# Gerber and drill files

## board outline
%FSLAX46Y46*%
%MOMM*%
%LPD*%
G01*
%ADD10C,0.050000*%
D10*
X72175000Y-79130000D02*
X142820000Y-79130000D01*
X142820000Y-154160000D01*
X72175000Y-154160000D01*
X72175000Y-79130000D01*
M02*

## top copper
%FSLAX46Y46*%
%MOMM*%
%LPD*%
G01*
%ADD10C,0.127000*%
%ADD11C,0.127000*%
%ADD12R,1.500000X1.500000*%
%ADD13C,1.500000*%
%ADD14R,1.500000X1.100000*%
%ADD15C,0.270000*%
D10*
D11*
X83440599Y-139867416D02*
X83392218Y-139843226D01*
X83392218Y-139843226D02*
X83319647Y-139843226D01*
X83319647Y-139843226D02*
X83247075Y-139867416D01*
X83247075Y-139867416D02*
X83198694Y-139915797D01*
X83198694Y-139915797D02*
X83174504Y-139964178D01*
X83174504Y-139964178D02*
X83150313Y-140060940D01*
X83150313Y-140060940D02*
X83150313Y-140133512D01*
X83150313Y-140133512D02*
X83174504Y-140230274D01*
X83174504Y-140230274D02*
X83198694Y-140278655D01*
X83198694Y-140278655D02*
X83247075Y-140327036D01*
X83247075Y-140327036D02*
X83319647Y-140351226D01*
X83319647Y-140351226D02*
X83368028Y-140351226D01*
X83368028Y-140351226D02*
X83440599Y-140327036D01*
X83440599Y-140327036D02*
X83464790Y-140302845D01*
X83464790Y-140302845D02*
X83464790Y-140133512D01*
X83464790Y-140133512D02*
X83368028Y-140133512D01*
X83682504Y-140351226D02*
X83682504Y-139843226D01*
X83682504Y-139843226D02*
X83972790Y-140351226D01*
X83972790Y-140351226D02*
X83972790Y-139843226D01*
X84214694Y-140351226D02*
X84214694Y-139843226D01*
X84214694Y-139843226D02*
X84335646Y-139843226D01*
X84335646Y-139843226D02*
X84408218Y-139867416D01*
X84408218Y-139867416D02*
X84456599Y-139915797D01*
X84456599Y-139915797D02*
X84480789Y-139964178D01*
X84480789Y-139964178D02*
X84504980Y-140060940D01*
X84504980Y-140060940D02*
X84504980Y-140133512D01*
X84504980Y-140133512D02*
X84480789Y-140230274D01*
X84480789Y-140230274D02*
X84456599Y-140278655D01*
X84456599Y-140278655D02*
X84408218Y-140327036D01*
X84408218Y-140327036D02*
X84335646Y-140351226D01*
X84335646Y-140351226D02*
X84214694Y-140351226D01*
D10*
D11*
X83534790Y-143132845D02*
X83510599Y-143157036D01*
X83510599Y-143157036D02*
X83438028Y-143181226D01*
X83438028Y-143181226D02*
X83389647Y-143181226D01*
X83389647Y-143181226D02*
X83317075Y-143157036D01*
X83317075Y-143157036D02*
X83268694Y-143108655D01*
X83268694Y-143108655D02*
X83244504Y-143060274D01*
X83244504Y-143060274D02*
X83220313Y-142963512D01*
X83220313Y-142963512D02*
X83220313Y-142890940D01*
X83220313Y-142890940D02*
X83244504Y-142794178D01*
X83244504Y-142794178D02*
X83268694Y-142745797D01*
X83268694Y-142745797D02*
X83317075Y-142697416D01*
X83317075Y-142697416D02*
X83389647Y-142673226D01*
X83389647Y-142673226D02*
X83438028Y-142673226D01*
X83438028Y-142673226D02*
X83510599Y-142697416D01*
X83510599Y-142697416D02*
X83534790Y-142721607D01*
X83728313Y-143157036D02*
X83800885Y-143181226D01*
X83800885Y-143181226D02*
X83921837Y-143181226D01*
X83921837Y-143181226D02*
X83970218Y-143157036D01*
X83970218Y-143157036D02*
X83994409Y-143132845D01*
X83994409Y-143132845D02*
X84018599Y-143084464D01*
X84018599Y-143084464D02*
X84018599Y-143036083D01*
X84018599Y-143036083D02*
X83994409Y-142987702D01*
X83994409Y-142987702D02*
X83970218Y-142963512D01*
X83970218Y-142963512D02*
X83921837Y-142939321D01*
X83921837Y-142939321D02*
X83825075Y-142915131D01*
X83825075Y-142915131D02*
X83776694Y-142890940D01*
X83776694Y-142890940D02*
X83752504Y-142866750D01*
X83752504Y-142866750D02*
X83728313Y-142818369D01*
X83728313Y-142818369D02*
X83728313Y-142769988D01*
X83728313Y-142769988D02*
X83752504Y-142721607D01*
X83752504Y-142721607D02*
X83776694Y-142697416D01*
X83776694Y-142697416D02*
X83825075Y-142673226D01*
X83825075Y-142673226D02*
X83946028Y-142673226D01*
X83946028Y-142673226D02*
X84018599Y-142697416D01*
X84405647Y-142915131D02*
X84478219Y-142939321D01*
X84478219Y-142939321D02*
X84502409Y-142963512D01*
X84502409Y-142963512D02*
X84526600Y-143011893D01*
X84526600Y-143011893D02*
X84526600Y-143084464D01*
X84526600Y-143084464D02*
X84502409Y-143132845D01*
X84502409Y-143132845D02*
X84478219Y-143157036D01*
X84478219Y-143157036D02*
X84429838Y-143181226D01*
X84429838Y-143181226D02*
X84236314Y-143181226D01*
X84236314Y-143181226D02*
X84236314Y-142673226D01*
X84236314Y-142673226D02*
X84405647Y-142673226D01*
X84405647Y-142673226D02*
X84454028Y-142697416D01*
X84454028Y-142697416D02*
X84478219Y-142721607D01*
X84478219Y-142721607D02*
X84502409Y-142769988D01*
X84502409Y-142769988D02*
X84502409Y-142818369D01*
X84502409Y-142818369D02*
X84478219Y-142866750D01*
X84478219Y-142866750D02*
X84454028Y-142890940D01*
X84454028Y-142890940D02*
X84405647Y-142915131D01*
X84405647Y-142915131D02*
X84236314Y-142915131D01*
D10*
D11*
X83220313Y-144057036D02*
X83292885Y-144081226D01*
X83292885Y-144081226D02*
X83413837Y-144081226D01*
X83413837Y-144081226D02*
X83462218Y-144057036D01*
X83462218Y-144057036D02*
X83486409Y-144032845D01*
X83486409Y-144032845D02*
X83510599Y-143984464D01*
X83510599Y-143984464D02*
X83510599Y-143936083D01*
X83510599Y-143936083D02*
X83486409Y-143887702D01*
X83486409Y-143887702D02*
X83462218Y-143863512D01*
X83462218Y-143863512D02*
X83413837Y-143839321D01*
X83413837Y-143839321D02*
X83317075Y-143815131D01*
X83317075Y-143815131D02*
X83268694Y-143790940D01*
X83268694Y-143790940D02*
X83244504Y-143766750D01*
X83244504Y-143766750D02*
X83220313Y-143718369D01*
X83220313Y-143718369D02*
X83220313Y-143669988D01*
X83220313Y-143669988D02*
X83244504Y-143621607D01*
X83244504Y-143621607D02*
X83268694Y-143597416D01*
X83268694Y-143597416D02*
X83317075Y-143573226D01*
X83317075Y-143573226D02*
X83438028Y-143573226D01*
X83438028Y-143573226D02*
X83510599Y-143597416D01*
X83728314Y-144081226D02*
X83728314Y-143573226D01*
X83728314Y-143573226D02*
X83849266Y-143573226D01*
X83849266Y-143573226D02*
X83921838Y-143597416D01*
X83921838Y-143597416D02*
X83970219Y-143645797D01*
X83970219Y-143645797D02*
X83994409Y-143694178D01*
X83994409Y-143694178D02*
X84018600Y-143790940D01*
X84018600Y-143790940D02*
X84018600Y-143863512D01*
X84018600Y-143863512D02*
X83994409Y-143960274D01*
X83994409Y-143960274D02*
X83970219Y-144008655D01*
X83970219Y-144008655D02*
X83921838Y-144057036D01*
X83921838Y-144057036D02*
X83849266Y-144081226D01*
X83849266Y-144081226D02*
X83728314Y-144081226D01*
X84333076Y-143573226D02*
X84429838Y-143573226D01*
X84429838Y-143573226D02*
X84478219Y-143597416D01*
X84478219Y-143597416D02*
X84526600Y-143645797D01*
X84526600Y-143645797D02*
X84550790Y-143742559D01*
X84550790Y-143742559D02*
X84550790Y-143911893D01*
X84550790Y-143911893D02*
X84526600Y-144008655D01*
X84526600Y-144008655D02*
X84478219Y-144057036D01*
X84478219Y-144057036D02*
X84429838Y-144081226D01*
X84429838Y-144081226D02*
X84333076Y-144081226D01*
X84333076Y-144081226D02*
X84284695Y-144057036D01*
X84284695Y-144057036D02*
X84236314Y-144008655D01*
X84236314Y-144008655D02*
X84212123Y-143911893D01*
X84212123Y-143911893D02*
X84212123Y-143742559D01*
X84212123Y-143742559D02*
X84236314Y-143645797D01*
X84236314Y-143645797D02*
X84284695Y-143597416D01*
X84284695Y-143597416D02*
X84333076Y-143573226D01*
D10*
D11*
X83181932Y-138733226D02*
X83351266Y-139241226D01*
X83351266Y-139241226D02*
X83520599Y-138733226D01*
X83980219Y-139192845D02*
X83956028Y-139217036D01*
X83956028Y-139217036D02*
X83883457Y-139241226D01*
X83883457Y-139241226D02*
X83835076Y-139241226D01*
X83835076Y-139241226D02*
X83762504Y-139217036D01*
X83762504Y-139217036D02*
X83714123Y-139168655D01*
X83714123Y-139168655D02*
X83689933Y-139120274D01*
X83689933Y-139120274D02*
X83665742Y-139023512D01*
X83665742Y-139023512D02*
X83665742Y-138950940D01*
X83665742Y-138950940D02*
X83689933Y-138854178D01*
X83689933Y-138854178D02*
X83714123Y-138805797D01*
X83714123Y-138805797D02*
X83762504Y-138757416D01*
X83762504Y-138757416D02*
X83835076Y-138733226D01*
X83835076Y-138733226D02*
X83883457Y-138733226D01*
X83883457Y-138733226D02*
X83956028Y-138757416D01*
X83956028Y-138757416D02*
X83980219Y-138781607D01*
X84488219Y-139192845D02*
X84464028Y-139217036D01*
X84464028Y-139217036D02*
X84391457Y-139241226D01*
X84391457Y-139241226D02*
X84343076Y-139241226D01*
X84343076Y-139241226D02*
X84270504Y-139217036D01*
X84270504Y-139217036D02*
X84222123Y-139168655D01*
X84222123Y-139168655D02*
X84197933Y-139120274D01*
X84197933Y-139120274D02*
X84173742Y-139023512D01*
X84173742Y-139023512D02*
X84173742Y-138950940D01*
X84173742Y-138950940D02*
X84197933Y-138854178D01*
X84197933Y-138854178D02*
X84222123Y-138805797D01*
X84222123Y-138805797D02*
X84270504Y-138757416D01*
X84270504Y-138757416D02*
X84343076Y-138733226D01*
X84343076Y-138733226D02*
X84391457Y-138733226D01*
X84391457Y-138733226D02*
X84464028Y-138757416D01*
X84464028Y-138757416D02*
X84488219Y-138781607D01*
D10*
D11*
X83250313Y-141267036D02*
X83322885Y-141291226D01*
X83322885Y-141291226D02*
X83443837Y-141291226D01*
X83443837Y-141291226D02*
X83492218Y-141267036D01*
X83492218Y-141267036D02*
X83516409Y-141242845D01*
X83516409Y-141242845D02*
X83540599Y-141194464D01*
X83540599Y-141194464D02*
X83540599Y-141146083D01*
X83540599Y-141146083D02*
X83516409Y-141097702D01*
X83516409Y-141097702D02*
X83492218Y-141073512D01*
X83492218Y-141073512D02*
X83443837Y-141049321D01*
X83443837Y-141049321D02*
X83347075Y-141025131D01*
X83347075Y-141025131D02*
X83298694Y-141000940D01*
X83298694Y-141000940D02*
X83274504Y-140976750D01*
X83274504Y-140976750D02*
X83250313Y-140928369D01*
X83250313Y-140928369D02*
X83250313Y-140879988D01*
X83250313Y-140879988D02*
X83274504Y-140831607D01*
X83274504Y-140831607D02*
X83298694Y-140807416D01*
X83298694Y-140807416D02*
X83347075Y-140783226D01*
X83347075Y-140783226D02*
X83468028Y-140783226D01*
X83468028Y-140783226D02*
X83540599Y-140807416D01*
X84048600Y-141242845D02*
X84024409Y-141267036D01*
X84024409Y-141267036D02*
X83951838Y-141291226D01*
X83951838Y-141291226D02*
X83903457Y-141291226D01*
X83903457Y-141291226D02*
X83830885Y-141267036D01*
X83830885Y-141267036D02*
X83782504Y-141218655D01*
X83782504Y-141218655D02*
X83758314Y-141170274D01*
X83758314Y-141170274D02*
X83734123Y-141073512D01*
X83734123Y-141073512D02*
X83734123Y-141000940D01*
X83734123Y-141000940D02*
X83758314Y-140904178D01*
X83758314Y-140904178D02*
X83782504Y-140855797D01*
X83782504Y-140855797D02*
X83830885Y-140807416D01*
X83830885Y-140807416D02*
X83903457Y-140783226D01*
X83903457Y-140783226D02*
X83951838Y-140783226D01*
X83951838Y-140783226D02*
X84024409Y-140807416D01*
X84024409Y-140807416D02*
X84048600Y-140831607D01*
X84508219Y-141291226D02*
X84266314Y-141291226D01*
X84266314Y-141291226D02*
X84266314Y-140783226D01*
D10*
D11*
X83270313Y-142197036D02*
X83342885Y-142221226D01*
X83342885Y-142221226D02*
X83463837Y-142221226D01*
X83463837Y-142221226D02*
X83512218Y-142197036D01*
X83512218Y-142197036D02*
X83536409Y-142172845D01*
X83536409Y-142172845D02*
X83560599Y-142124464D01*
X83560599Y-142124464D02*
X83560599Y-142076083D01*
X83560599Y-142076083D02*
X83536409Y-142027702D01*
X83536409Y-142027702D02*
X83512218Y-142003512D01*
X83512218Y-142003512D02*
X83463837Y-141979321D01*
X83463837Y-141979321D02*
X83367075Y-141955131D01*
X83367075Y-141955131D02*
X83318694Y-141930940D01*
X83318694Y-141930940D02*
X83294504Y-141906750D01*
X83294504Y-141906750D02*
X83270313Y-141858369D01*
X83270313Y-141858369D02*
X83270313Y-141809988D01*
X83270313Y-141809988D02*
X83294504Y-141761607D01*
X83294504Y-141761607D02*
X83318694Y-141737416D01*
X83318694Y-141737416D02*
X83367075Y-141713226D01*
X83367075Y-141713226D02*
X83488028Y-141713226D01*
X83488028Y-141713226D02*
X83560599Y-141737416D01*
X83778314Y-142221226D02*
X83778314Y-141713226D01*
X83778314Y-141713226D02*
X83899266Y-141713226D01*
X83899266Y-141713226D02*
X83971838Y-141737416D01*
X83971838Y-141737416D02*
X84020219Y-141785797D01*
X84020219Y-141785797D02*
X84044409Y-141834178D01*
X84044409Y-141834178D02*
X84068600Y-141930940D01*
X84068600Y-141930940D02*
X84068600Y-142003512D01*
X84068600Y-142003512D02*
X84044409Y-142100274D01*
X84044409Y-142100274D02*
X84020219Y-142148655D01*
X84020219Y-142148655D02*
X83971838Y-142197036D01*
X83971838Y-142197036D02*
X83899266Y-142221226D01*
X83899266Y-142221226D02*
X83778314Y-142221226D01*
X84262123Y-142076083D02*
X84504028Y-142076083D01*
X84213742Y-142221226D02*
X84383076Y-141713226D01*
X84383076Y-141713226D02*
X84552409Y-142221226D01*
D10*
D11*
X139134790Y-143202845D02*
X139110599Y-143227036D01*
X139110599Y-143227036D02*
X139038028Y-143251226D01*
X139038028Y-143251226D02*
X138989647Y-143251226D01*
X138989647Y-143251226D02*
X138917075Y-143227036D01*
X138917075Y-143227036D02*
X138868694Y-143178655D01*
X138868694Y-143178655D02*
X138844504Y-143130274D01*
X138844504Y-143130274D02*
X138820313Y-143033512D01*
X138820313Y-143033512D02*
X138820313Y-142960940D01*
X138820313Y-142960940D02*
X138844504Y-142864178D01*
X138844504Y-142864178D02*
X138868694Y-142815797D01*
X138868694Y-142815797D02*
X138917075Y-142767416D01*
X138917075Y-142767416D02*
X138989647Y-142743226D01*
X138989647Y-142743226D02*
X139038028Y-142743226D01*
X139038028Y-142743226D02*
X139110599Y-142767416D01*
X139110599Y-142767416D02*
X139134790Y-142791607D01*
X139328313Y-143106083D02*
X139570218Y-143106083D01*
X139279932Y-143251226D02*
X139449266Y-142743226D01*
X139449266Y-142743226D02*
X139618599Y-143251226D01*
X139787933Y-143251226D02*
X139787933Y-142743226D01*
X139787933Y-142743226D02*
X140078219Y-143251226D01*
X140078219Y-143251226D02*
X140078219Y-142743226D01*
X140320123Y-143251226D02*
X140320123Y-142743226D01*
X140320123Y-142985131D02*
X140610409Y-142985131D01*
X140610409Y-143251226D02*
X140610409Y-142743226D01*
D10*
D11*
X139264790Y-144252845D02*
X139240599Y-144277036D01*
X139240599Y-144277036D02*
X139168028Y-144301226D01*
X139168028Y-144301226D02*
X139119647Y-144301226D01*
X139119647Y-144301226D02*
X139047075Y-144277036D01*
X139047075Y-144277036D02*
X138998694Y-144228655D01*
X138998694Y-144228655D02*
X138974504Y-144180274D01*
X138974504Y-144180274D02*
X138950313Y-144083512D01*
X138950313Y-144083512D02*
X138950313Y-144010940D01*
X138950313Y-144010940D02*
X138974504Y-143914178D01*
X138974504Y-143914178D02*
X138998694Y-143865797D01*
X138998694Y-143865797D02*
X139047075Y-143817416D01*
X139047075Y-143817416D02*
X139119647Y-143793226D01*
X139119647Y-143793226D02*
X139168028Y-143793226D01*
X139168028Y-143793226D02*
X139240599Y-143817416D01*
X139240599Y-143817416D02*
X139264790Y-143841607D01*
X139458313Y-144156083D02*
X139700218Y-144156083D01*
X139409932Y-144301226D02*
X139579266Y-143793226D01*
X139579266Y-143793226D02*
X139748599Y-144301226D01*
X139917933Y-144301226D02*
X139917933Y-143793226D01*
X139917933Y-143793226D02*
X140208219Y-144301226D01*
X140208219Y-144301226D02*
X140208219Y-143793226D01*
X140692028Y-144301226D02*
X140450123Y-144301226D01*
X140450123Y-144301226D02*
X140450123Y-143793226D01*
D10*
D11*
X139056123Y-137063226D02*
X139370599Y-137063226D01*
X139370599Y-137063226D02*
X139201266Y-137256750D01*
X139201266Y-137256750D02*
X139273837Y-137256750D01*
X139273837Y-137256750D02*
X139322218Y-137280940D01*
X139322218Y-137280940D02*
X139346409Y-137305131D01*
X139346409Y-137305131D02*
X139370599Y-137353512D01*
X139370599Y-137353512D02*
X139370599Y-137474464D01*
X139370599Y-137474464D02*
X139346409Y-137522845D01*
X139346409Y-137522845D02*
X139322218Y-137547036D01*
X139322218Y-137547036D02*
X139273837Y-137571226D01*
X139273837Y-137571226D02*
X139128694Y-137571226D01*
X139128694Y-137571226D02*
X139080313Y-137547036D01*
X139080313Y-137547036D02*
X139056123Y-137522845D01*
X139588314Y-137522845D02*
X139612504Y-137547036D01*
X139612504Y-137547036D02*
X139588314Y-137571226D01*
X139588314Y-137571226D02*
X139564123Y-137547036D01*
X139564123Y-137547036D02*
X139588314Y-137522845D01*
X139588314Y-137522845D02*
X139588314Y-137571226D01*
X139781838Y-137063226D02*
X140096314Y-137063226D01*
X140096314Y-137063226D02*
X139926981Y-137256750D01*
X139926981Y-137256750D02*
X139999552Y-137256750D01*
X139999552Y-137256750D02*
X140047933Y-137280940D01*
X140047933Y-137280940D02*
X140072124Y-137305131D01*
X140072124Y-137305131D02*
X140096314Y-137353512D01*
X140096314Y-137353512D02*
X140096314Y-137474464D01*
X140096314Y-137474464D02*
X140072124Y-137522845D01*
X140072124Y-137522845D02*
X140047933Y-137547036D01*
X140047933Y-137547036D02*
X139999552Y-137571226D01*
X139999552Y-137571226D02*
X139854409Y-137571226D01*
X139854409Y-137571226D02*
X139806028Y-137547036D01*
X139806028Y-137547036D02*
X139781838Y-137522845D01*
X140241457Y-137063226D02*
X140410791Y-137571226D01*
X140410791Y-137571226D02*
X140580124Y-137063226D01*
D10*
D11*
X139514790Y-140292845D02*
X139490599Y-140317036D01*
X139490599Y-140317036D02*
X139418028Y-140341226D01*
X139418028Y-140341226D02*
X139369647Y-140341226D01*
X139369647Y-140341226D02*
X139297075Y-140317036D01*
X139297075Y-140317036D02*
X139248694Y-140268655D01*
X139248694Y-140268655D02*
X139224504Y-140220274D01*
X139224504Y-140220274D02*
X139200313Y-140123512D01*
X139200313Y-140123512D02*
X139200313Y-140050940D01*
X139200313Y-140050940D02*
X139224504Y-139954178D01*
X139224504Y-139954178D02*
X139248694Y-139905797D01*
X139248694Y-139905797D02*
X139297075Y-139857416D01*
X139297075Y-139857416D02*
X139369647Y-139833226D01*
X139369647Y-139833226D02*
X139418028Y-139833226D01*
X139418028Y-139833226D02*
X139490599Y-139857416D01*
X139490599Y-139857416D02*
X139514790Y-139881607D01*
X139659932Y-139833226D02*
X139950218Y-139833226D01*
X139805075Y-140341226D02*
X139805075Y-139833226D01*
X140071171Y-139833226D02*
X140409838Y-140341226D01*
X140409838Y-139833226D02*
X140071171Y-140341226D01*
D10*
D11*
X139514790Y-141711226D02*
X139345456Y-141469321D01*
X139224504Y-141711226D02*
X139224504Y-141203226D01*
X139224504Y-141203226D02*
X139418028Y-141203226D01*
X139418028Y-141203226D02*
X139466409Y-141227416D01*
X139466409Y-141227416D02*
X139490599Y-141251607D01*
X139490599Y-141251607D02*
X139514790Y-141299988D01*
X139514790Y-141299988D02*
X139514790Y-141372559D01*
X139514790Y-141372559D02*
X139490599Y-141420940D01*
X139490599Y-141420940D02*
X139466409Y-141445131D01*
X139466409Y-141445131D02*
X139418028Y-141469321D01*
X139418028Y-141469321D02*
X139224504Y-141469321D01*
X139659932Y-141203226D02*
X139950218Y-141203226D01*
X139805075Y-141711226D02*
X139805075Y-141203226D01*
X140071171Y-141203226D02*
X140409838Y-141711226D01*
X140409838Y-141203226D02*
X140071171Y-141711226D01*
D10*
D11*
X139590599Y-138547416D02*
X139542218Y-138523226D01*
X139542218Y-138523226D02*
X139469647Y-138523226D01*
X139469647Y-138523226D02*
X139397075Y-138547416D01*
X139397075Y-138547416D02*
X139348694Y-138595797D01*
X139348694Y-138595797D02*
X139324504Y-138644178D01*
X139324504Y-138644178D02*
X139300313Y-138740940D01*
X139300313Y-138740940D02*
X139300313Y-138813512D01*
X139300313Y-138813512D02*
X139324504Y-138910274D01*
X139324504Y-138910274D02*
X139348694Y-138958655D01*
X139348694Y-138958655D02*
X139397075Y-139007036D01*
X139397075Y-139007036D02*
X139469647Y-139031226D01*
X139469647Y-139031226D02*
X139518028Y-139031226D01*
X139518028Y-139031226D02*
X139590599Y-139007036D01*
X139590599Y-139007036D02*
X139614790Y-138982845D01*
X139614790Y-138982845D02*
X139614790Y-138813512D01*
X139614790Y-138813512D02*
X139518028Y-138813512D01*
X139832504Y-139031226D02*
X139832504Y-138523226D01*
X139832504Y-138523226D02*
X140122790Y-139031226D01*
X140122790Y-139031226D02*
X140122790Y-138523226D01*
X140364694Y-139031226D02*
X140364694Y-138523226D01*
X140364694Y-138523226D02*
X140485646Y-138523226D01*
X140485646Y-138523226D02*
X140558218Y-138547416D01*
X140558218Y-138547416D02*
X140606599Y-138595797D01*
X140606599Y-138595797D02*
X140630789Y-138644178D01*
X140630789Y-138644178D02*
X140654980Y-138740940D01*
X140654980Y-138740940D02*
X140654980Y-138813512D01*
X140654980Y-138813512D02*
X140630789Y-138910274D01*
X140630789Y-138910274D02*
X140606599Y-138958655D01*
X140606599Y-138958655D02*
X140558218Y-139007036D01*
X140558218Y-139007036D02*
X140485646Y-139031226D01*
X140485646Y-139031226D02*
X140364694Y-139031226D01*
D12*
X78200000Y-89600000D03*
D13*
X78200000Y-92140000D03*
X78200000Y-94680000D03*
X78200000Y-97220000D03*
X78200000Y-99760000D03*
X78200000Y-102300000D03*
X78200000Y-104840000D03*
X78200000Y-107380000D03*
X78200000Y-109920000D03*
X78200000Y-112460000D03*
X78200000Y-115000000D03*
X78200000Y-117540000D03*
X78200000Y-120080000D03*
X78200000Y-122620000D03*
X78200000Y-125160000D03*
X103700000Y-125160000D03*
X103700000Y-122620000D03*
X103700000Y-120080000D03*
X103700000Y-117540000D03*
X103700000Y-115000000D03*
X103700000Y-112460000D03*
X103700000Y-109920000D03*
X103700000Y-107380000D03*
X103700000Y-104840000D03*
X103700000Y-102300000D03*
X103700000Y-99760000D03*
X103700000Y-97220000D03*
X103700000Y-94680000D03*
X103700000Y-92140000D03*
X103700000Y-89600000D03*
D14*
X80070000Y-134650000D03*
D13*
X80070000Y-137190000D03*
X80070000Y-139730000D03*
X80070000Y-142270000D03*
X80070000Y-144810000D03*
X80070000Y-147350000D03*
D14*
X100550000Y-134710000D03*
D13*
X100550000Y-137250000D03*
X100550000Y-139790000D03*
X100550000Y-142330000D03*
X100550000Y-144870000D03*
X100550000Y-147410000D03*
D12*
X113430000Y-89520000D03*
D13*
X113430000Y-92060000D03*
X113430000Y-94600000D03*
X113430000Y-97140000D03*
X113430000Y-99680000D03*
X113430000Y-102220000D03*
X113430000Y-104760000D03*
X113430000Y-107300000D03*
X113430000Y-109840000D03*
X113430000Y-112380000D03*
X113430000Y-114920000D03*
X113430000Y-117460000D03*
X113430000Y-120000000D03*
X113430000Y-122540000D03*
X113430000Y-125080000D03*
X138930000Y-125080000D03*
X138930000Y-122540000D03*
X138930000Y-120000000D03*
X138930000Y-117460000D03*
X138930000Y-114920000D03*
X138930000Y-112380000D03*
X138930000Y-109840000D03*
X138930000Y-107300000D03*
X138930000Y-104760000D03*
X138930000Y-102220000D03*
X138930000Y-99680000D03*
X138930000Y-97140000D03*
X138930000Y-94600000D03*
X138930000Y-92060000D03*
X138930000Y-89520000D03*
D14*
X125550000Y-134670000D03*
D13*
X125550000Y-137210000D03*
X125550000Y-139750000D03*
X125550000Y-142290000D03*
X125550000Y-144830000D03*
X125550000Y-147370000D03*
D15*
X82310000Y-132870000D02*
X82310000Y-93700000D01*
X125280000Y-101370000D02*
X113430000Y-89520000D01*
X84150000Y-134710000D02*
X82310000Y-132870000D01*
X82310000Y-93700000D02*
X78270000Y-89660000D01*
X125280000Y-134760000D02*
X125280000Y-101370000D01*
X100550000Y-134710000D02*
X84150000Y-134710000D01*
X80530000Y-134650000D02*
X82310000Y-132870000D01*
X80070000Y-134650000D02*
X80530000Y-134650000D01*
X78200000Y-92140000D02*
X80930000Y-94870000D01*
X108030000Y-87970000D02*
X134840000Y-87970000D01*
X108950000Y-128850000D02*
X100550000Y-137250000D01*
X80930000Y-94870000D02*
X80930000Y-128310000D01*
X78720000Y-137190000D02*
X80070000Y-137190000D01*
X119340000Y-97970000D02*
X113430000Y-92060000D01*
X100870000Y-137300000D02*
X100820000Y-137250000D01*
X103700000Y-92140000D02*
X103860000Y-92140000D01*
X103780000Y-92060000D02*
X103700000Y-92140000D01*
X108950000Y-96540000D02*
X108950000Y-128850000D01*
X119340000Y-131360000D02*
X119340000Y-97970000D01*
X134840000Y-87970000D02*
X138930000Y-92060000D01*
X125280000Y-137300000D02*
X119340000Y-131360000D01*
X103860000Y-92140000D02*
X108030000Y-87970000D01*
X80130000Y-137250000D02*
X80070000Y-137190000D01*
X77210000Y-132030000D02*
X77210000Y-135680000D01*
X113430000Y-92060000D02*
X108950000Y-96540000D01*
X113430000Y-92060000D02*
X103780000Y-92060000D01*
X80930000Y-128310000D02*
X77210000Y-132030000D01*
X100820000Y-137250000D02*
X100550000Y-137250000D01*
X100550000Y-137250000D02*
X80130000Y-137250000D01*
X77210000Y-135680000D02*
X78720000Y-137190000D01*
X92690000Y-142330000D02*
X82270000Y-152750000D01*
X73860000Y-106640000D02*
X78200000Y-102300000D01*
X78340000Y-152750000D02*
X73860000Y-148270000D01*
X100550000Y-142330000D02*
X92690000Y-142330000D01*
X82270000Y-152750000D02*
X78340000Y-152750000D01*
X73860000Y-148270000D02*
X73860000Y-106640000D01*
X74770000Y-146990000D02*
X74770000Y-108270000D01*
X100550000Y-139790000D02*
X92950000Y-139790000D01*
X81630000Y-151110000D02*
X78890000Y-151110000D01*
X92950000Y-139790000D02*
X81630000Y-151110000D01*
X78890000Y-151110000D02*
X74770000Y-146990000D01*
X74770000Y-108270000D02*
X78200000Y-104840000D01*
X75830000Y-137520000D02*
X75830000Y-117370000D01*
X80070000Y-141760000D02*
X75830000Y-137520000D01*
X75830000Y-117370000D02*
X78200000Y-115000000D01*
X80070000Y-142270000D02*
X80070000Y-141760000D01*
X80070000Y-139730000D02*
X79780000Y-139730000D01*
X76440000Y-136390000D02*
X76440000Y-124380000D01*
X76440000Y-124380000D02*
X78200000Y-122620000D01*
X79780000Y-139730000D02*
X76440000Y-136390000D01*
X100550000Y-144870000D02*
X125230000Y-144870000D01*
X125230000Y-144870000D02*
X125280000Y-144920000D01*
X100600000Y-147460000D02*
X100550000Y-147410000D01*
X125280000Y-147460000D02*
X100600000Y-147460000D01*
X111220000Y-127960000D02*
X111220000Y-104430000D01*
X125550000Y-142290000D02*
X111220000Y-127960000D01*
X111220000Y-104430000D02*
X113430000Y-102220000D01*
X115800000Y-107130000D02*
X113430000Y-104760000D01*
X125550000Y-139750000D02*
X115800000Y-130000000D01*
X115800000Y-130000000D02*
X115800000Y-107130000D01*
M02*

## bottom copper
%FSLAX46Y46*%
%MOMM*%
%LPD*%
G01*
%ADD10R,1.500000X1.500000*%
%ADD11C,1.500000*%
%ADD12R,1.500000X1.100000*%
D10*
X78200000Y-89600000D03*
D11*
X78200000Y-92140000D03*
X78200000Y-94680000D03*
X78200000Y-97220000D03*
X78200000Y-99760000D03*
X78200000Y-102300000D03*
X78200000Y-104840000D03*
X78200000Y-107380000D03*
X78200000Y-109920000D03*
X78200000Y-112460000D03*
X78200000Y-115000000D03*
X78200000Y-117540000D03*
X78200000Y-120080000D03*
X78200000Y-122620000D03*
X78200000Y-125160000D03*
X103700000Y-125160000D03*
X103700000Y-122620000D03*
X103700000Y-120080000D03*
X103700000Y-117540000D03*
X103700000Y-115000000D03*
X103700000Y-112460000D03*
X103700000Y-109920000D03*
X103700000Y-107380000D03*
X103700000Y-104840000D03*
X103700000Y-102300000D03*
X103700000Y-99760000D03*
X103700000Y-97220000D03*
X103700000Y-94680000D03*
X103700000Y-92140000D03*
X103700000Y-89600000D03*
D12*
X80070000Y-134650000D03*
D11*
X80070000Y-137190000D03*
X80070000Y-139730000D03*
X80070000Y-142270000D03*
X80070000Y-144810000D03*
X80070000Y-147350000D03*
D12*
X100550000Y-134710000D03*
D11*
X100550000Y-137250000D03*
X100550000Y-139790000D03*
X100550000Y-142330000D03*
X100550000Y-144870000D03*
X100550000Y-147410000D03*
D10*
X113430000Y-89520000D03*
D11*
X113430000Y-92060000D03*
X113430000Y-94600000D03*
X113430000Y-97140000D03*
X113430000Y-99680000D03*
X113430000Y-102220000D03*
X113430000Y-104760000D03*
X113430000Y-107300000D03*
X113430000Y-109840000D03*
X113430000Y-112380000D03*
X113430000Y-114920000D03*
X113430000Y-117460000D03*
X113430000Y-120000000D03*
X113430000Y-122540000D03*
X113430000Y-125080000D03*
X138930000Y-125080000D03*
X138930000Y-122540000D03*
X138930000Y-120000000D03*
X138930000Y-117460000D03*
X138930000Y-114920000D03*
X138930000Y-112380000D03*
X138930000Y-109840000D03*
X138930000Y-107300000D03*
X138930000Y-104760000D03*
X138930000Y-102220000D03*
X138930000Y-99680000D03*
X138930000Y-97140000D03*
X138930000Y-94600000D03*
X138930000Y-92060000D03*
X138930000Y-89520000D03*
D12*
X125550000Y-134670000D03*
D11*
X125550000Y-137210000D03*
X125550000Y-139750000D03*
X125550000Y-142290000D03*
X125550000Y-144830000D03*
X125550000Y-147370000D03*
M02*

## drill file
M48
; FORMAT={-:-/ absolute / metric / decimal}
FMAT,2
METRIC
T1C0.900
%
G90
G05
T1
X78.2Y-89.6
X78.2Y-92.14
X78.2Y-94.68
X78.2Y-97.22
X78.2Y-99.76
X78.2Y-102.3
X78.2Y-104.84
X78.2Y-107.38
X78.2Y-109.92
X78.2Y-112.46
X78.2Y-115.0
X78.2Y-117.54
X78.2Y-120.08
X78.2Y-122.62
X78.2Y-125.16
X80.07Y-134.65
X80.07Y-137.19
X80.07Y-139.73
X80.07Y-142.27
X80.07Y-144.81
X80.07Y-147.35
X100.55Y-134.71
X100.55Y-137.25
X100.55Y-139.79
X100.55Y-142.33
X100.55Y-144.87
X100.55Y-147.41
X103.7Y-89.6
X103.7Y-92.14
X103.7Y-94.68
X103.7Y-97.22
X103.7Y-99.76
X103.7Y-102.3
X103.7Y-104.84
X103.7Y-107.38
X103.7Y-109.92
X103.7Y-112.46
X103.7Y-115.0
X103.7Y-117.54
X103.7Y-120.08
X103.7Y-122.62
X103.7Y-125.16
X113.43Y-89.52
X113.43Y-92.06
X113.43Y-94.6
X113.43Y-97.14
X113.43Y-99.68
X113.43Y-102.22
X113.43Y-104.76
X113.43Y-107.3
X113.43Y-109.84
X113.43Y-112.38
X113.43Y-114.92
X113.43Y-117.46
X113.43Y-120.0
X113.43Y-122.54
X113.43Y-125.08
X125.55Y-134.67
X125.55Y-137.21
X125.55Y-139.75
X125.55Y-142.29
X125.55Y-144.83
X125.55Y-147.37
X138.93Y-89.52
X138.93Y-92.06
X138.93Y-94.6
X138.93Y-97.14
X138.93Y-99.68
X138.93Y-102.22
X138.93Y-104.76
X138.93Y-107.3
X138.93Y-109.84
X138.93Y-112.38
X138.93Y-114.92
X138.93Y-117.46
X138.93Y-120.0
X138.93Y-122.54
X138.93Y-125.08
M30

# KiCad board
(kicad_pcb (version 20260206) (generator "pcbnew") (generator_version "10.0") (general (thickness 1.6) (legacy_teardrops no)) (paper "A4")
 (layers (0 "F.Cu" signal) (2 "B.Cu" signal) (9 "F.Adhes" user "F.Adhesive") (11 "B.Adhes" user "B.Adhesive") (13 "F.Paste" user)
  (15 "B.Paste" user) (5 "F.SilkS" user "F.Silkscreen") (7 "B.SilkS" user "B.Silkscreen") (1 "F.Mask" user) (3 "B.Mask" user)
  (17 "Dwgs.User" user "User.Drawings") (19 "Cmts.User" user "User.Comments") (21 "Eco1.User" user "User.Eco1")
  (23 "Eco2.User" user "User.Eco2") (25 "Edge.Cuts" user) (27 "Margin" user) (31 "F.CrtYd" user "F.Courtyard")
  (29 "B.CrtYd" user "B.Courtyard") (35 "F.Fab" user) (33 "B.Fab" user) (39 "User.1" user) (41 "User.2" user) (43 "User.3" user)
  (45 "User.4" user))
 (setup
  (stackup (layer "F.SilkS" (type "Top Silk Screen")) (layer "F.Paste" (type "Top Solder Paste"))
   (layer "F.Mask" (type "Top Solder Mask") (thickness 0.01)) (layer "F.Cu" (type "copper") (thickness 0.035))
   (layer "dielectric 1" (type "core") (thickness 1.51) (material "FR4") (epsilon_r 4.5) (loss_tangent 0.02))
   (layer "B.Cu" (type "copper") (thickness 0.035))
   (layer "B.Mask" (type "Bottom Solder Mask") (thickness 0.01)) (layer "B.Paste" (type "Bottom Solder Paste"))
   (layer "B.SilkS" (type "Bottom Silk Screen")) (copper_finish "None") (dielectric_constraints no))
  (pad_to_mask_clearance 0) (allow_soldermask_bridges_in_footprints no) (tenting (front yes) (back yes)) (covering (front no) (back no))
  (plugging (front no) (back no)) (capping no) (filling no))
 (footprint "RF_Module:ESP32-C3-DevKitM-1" (layer "F.Cu") (at 78.2 89.6)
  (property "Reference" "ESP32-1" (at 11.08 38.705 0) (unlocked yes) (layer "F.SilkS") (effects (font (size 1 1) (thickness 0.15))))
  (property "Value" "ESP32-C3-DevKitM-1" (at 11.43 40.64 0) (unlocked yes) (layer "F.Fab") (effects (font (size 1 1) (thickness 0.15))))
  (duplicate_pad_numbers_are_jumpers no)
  (pad "1" thru_hole rect (at 0 0) (size 1.5 1.5) (drill 0.9) (layers "*.Cu" "*.Mask") (remove_unused_layers yes) (keep_end_layers yes)
   (zone_layer_connections) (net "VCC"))
  (pad "2" thru_hole circle (at 0 2.54) (size 1.5 1.5) (drill 0.9) (layers "*.Cu" "*.Mask") (remove_unused_layers yes) (keep_end_layers yes)
   (zone_layer_connections) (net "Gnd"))
  (pad "3" thru_hole circle (at 0 5.08) (size 1.5 1.5) (drill 0.9) (layers "*.Cu" "*.Mask") (remove_unused_layers yes) (keep_end_layers yes)
   (zone_layer_connections))
  (pad "4" thru_hole circle (at 0 7.62) (size 1.5 1.5) (drill 0.9) (layers "*.Cu" "*.Mask") (remove_unused_layers yes) (keep_end_layers yes)
   (zone_layer_connections))
  (pad "5" thru_hole circle (at 0 10.16) (size 1.5 1.5) (drill 0.9) (layers "*.Cu" "*.Mask") (remove_unused_layers yes)
   (keep_end_layers yes) (zone_layer_connections))
  (pad "6" thru_hole circle (at 0 12.7) (size 1.5 1.5) (drill 0.9) (layers "*.Cu" "*.Mask") (remove_unused_layers yes) (keep_end_layers yes)
   (zone_layer_connections) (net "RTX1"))
  (pad "7" thru_hole circle (at 0 15.24) (size 1.5 1.5) (drill 0.9) (layers "*.Cu" "*.Mask") (remove_unused_layers yes)
   (keep_end_layers yes) (zone_layer_connections) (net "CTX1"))
  (pad "8" thru_hole circle (at 0 17.78) (size 1.5 1.5) (drill 0.9) (layers "*.Cu" "*.Mask") (remove_unused_layers yes)
   (keep_end_layers yes) (zone_layer_connections))
  (pad "9" thru_hole circle (at 0 20.32) (size 1.5 1.5) (drill 0.9) (layers "*.Cu" "*.Mask") (remove_unused_layers yes)
   (keep_end_layers yes) (zone_layer_connections))
  (pad "10" thru_hole circle (at 0 22.86) (size 1.5 1.5) (drill 0.9) (layers "*.Cu" "*.Mask") (remove_unused_layers yes)
   (keep_end_layers yes) (zone_layer_connections))
  (pad "11" thru_hole circle (at 0 25.4) (size 1.5 1.5) (drill 0.9) (layers "*.Cu" "*.Mask") (remove_unused_layers yes)
   (keep_end_layers yes) (zone_layer_connections) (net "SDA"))
  (pad "12" thru_hole circle (at 0 27.94) (size 1.5 1.5) (drill 0.9) (layers "*.Cu" "*.Mask") (remove_unused_layers yes)
   (keep_end_layers yes) (zone_layer_connections))
  (pad "13" thru_hole circle (at 0 30.48) (size 1.5 1.5) (drill 0.9) (layers "*.Cu" "*.Mask") (remove_unused_layers yes)
   (keep_end_layers yes) (zone_layer_connections))
  (pad "14" thru_hole circle (at 0 33.02) (size 1.5 1.5) (drill 0.9) (layers "*.Cu" "*.Mask") (remove_unused_layers yes)
   (keep_end_layers yes) (zone_layer_connections) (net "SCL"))
  (pad "15" thru_hole circle (at 0 35.56) (size 1.5 1.5) (drill 0.9) (layers "*.Cu" "*.Mask") (remove_unused_layers yes)
   (keep_end_layers yes) (zone_layer_connections))
  (pad "16" thru_hole circle (at 25.5 35.56) (size 1.5 1.5) (drill 0.9) (layers "*.Cu" "*.Mask") (remove_unused_layers yes)
   (keep_end_layers yes) (zone_layer_connections))
  (pad "17" thru_hole circle (at 25.5 33.02) (size 1.5 1.5) (drill 0.9) (layers "*.Cu" "*.Mask") (remove_unused_layers yes)
   (keep_end_layers yes) (zone_layer_connections))
  (pad "18" thru_hole circle (at 25.5 30.48) (size 1.5 1.5) (drill 0.9) (layers "*.Cu" "*.Mask") (remove_unused_layers yes)
   (keep_end_layers yes) (zone_layer_connections))
  (pad "19" thru_hole circle (at 25.5 27.94) (size 1.5 1.5) (drill 0.9) (layers "*.Cu" "*.Mask") (remove_unused_layers yes)
   (keep_end_layers yes) (zone_layer_connections))
  (pad "20" thru_hole circle (at 25.5 25.4) (size 1.5 1.5) (drill 0.9) (layers "*.Cu" "*.Mask") (remove_unused_layers yes)
   (keep_end_layers yes) (zone_layer_connections))
  (pad "21" thru_hole circle (at 25.5 22.86) (size 1.5 1.5) (drill 0.9) (layers "*.Cu" "*.Mask") (remove_unused_layers yes)
   (keep_end_layers yes) (zone_layer_connections))
  (pad "22" thru_hole circle (at 25.5 20.32) (size 1.5 1.5) (drill 0.9) (layers "*.Cu" "*.Mask") (remove_unused_layers yes)
   (keep_end_layers yes) (zone_layer_connections))
  (pad "23" thru_hole circle (at 25.5 17.78) (size 1.5 1.5) (drill 0.9) (layers "*.Cu" "*.Mask") (remove_unused_layers yes)
   (keep_end_layers yes) (zone_layer_connections))
  (pad "24" thru_hole circle (at 25.5 15.24) (size 1.5 1.5) (drill 0.9) (layers "*.Cu" "*.Mask") (remove_unused_layers yes)
   (keep_end_layers yes) (zone_layer_connections))
  (pad "25" thru_hole circle (at 25.5 12.7) (size 1.5 1.5) (drill 0.9) (layers "*.Cu" "*.Mask") (remove_unused_layers yes)
   (keep_end_layers yes) (zone_layer_connections))
  (pad "26" thru_hole circle (at 25.5 10.16) (size 1.5 1.5) (drill 0.9) (layers "*.Cu" "*.Mask") (remove_unused_layers yes)
   (keep_end_layers yes) (zone_layer_connections))
  (pad "27" thru_hole circle (at 25.5 7.62) (size 1.5 1.5) (drill 0.9) (layers "*.Cu" "*.Mask") (remove_unused_layers yes)
   (keep_end_layers yes) (zone_layer_connections))
  (pad "28" thru_hole circle (at 25.5 5.08) (size 1.5 1.5) (drill 0.9) (layers "*.Cu" "*.Mask") (remove_unused_layers yes)
   (keep_end_layers yes) (zone_layer_connections))
  (pad "29" thru_hole circle (at 25.5 2.54) (size 1.5 1.5) (drill 0.9) (layers "*.Cu" "*.Mask") (remove_unused_layers yes)
   (keep_end_layers yes) (zone_layer_connections) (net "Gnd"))
  (pad "30" thru_hole circle (at 25.5 0) (size 1.5 1.5) (drill 0.9) (layers "*.Cu" "*.Mask") (remove_unused_layers yes)
   (keep_end_layers yes) (zone_layer_connections)))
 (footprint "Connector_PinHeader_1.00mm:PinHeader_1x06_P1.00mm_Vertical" (layer "F.Cu") (at 80.07 134.65)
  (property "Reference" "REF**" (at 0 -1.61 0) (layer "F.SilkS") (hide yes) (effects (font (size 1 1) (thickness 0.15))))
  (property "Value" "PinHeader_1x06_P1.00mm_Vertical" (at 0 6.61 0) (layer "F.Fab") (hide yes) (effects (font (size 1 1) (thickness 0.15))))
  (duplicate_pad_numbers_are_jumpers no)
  (pad "1" thru_hole rect (at 0 0) (size 1.5 1.1) (drill 0.9) (layers "*.Cu" "*.Mask") (remove_unused_layers no) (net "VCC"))
  (pad "2" thru_hole circle (at 0 2.54) (size 1.5 1.5) (drill 0.9) (layers "*.Cu" "*.Mask") (remove_unused_layers no) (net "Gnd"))
  (pad "3" thru_hole circle (at 0 5.08) (size 1.5 1.5) (drill 0.9) (layers "*.Cu" "*.Mask") (remove_unused_layers no) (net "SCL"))
  (pad "4" thru_hole circle (at 0 7.62) (size 1.5 1.5) (drill 0.9) (layers "*.Cu" "*.Mask") (remove_unused_layers no) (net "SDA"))
  (pad "5" thru_hole circle (at 0 10.16) (size 1.5 1.5) (drill 0.9) (layers "*.Cu" "*.Mask") (remove_unused_layers no))
  (pad "6" thru_hole circle (at 0 12.7) (size 1.5 1.5) (drill 0.9) (layers "*.Cu" "*.Mask") (remove_unused_layers no)))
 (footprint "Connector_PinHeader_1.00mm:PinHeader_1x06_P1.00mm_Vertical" (layer "F.Cu") (at 100.55 134.71)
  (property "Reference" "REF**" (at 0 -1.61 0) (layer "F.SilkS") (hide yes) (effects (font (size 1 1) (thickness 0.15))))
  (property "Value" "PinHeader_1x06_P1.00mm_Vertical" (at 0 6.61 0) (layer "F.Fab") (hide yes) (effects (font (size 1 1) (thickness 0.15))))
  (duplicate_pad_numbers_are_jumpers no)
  (pad "1" thru_hole rect (at 0 0) (size 1.5 1.1) (drill 0.9) (layers "*.Cu" "*.Mask") (remove_unused_layers no) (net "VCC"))
  (pad "2" thru_hole circle (at 0 2.54) (size 1.5 1.5) (drill 0.9) (layers "*.Cu" "*.Mask") (remove_unused_layers no) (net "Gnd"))
  (pad "3" thru_hole circle (at 0 5.08) (size 1.5 1.5) (drill 0.9) (layers "*.Cu" "*.Mask") (remove_unused_layers no) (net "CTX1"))
  (pad "4" thru_hole circle (at 0 7.62) (size 1.5 1.5) (drill 0.9) (layers "*.Cu" "*.Mask") (remove_unused_layers no) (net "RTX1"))
  (pad "5" thru_hole circle (at 0 10.16) (size 1.5 1.5) (drill 0.9) (layers "*.Cu" "*.Mask") (remove_unused_layers no) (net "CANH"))
  (pad "6" thru_hole circle (at 0 12.7) (size 1.5 1.5) (drill 0.9) (layers "*.Cu" "*.Mask") (remove_unused_layers no) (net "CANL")))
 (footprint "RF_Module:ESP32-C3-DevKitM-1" (layer "F.Cu") (at 113.43 89.52)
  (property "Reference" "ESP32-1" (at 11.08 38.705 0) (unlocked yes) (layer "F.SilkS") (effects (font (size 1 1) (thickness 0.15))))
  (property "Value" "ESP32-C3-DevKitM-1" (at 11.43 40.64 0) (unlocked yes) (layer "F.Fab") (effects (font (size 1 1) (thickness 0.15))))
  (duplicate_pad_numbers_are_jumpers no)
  (pad "1" thru_hole rect (at 0 0) (size 1.5 1.5) (drill 0.9) (layers "*.Cu" "*.Mask") (remove_unused_layers yes) (keep_end_layers yes)
   (zone_layer_connections) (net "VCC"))
  (pad "2" thru_hole circle (at 0 2.54) (size 1.5 1.5) (drill 0.9) (layers "*.Cu" "*.Mask") (remove_unused_layers yes) (keep_end_layers yes)
   (zone_layer_connections) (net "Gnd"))
  (pad "3" thru_hole circle (at 0 5.08) (size 1.5 1.5) (drill 0.9) (layers "*.Cu" "*.Mask") (remove_unused_layers yes) (keep_end_layers yes)
   (zone_layer_connections))
  (pad "4" thru_hole circle (at 0 7.62) (size 1.5 1.5) (drill 0.9) (layers "*.Cu" "*.Mask") (remove_unused_layers yes) (keep_end_layers yes)
   (zone_layer_connections))
  (pad "5" thru_hole circle (at 0 10.16) (size 1.5 1.5) (drill 0.9) (layers "*.Cu" "*.Mask") (remove_unused_layers yes)
   (keep_end_layers yes) (zone_layer_connections))
  (pad "6" thru_hole circle (at 0 12.7) (size 1.5 1.5) (drill 0.9) (layers "*.Cu" "*.Mask") (remove_unused_layers yes) (keep_end_layers yes)
   (zone_layer_connections) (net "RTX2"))
  (pad "7" thru_hole circle (at 0 15.24) (size 1.5 1.5) (drill 0.9) (layers "*.Cu" "*.Mask") (remove_unused_layers yes)
   (keep_end_layers yes) (zone_layer_connections) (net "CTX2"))
  (pad "8" thru_hole circle (at 0 17.78) (size 1.5 1.5) (drill 0.9) (layers "*.Cu" "*.Mask") (remove_unused_layers yes)
   (keep_end_layers yes) (zone_layer_connections))
  (pad "9" thru_hole circle (at 0 20.32) (size 1.5 1.5) (drill 0.9) (layers "*.Cu" "*.Mask") (remove_unused_layers yes)
   (keep_end_layers yes) (zone_layer_connections))
  (pad "10" thru_hole circle (at 0 22.86) (size 1.5 1.5) (drill 0.9) (layers "*.Cu" "*.Mask") (remove_unused_layers yes)
   (keep_end_layers yes) (zone_layer_connections))
  (pad "11" thru_hole circle (at 0 25.4) (size 1.5 1.5) (drill 0.9) (layers "*.Cu" "*.Mask") (remove_unused_layers yes)
   (keep_end_layers yes) (zone_layer_connections))
  (pad "12" thru_hole circle (at 0 27.94) (size 1.5 1.5) (drill 0.9) (layers "*.Cu" "*.Mask") (remove_unused_layers yes)
   (keep_end_layers yes) (zone_layer_connections))
  (pad "13" thru_hole circle (at 0 30.48) (size 1.5 1.5) (drill 0.9) (layers "*.Cu" "*.Mask") (remove_unused_layers yes)
   (keep_end_layers yes) (zone_layer_connections))
  (pad "14" thru_hole circle (at 0 33.02) (size 1.5 1.5) (drill 0.9) (layers "*.Cu" "*.Mask") (remove_unused_layers yes)
   (keep_end_layers yes) (zone_layer_connections))
  (pad "15" thru_hole circle (at 0 35.56) (size 1.5 1.5) (drill 0.9) (layers "*.Cu" "*.Mask") (remove_unused_layers yes)
   (keep_end_layers yes) (zone_layer_connections))
  (pad "16" thru_hole circle (at 25.5 35.56) (size 1.5 1.5) (drill 0.9) (layers "*.Cu" "*.Mask") (remove_unused_layers yes)
   (keep_end_layers yes) (zone_layer_connections))
  (pad "17" thru_hole circle (at 25.5 33.02) (size 1.5 1.5) (drill 0.9) (layers "*.Cu" "*.Mask") (remove_unused_layers yes)
   (keep_end_layers yes) (zone_layer_connections))
  (pad "18" thru_hole circle (at 25.5 30.48) (size 1.5 1.5) (drill 0.9) (layers "*.Cu" "*.Mask") (remove_unused_layers yes)
   (keep_end_layers yes) (zone_layer_connections))
  (pad "19" thru_hole circle (at 25.5 27.94) (size 1.5 1.5) (drill 0.9) (layers "*.Cu" "*.Mask") (remove_unused_layers yes)
   (keep_end_layers yes) (zone_layer_connections))
  (pad "20" thru_hole circle (at 25.5 25.4) (size 1.5 1.5) (drill 0.9) (layers "*.Cu" "*.Mask") (remove_unused_layers yes)
   (keep_end_layers yes) (zone_layer_connections))
  (pad "21" thru_hole circle (at 25.5 22.86) (size 1.5 1.5) (drill 0.9) (layers "*.Cu" "*.Mask") (remove_unused_layers yes)
   (keep_end_layers yes) (zone_layer_connections))
  (pad "22" thru_hole circle (at 25.5 20.32) (size 1.5 1.5) (drill 0.9) (layers "*.Cu" "*.Mask") (remove_unused_layers yes)
   (keep_end_layers yes) (zone_layer_connections))
  (pad "23" thru_hole circle (at 25.5 17.78) (size 1.5 1.5) (drill 0.9) (layers "*.Cu" "*.Mask") (remove_unused_layers yes)
   (keep_end_layers yes) (zone_layer_connections))
  (pad "24" thru_hole circle (at 25.5 15.24) (size 1.5 1.5) (drill 0.9) (layers "*.Cu" "*.Mask") (remove_unused_layers yes)
   (keep_end_layers yes) (zone_layer_connections))
  (pad "25" thru_hole circle (at 25.5 12.7) (size 1.5 1.5) (drill 0.9) (layers "*.Cu" "*.Mask") (remove_unused_layers yes)
   (keep_end_layers yes) (zone_layer_connections))
  (pad "26" thru_hole circle (at 25.5 10.16) (size 1.5 1.5) (drill 0.9) (layers "*.Cu" "*.Mask") (remove_unused_layers yes)
   (keep_end_layers yes) (zone_layer_connections))
  (pad "27" thru_hole circle (at 25.5 7.62) (size 1.5 1.5) (drill 0.9) (layers "*.Cu" "*.Mask") (remove_unused_layers yes)
   (keep_end_layers yes) (zone_layer_connections))
  (pad "28" thru_hole circle (at 25.5 5.08) (size 1.5 1.5) (drill 0.9) (layers "*.Cu" "*.Mask") (remove_unused_layers yes)
   (keep_end_layers yes) (zone_layer_connections))
  (pad "29" thru_hole circle (at 25.5 2.54) (size 1.5 1.5) (drill 0.9) (layers "*.Cu" "*.Mask") (remove_unused_layers yes)
   (keep_end_layers yes) (zone_layer_connections) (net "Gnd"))
  (pad "30" thru_hole circle (at 25.5 0) (size 1.5 1.5) (drill 0.9) (layers "*.Cu" "*.Mask") (remove_unused_layers yes)
   (keep_end_layers yes) (zone_layer_connections)))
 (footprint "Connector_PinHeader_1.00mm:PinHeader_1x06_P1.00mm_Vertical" (layer "F.Cu") (at 125.55 134.67)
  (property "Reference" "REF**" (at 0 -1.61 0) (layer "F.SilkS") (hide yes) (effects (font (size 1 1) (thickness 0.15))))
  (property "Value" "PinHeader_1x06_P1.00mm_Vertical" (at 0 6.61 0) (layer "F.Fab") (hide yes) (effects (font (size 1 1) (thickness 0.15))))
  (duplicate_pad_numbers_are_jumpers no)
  (pad "1" thru_hole rect (at 0 0) (size 1.5 1.1) (drill 0.9) (layers "*.Cu" "*.Mask") (remove_unused_layers no) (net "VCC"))
  (pad "2" thru_hole circle (at 0 2.54) (size 1.5 1.5) (drill 0.9) (layers "*.Cu" "*.Mask") (remove_unused_layers no) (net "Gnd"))
  (pad "3" thru_hole circle (at 0 5.08) (size 1.5 1.5) (drill 0.9) (layers "*.Cu" "*.Mask") (remove_unused_layers no) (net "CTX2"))
  (pad "4" thru_hole circle (at 0 7.62) (size 1.5 1.5) (drill 0.9) (layers "*.Cu" "*.Mask") (remove_unused_layers no) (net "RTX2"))
  (pad "5" thru_hole circle (at 0 10.16) (size 1.5 1.5) (drill 0.9) (layers "*.Cu" "*.Mask") (remove_unused_layers no) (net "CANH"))
  (pad "6" thru_hole circle (at 0 12.7) (size 1.5 1.5) (drill 0.9) (layers "*.Cu" "*.Mask") (remove_unused_layers no) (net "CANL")))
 (gr_rect (start 72.175 79.13) (end 142.82 154.16) (stroke (width 0.05) (type default)) (fill no) (layer "Edge.Cuts"))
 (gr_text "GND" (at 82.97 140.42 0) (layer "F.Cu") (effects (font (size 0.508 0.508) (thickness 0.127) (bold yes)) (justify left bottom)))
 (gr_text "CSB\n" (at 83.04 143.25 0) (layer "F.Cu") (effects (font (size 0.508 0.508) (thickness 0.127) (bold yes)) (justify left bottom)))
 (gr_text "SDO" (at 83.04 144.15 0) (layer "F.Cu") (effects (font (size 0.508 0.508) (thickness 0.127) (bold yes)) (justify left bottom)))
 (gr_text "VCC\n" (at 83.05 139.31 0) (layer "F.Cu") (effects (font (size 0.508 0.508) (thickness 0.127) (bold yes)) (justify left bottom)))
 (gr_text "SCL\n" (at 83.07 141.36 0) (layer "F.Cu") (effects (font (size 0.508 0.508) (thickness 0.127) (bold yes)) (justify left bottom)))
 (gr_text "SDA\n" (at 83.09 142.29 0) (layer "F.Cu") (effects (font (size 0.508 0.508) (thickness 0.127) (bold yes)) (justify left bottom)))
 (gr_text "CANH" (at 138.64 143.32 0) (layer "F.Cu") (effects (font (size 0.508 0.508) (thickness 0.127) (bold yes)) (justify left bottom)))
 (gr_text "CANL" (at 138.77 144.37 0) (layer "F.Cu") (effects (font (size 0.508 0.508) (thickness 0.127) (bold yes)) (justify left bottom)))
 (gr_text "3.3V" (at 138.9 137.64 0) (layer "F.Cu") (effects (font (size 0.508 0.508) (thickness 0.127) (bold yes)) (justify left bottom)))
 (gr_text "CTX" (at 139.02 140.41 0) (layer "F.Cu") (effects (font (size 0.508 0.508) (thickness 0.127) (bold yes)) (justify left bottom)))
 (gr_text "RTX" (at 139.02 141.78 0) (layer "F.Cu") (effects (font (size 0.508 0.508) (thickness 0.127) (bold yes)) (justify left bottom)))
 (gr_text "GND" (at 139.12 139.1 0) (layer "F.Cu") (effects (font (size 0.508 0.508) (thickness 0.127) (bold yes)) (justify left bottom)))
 (segment (start 82.31 132.87) (end 82.31 93.7) (width 0.27) (layer "F.Cu") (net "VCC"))
 (segment (start 125.28 101.37) (end 113.43 89.52) (width 0.27) (layer "F.Cu") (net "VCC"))
 (segment (start 84.15 134.71) (end 82.31 132.87) (width 0.27) (layer "F.Cu") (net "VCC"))
 (segment (start 82.31 93.7) (end 78.27 89.66) (width 0.27) (layer "F.Cu") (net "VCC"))
 (segment (start 125.28 134.76) (end 125.28 101.37) (width 0.27) (layer "F.Cu") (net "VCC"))
 (segment (start 100.55 134.71) (end 84.15 134.71) (width 0.27) (layer "F.Cu") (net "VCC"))
 (segment (start 80.53 134.65) (end 82.31 132.87) (width 0.27) (layer "F.Cu") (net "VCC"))
 (segment (start 80.07 134.65) (end 80.53 134.65) (width 0.27) (layer "F.Cu") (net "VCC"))
 (segment (start 78.2 92.14) (end 80.93 94.87) (width 0.27) (layer "F.Cu") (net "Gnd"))
 (segment (start 108.03 87.97) (end 134.84 87.97) (width 0.27) (layer "F.Cu") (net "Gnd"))
 (segment (start 108.95 128.85) (end 100.55 137.25) (width 0.27) (layer "F.Cu") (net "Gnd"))
 (segment (start 80.93 94.87) (end 80.93 128.31) (width 0.27) (layer "F.Cu") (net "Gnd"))
 (segment (start 78.72 137.19) (end 80.07 137.19) (width 0.27) (layer "F.Cu") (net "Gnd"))
 (segment (start 119.34 97.97) (end 113.43 92.06) (width 0.27) (layer "F.Cu") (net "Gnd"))
 (segment (start 100.87 137.3) (end 100.82 137.25) (width 0.27) (layer "F.Cu") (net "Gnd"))
 (segment (start 103.7 92.14) (end 103.86 92.14) (width 0.27) (layer "F.Cu") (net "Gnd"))
 (segment (start 103.78 92.06) (end 103.7 92.14) (width 0.27) (layer "F.Cu") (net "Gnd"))
 (segment (start 108.95 96.54) (end 108.95 128.85) (width 0.27) (layer "F.Cu") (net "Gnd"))
 (segment (start 119.34 131.36) (end 119.34 97.97) (width 0.27) (layer "F.Cu") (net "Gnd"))
 (segment (start 134.84 87.97) (end 138.93 92.06) (width 0.27) (layer "F.Cu") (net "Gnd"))
 (segment (start 125.28 137.3) (end 119.34 131.36) (width 0.27) (layer "F.Cu") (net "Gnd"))
 (segment (start 103.86 92.14) (end 108.03 87.97) (width 0.27) (layer "F.Cu") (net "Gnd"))
 (segment (start 80.13 137.25) (end 80.07 137.19) (width 0.27) (layer "F.Cu") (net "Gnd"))
 (segment (start 77.21 132.03) (end 77.21 135.68) (width 0.27) (layer "F.Cu") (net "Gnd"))
 (segment (start 113.43 92.06) (end 108.95 96.54) (width 0.27) (layer "F.Cu") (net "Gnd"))
 (segment (start 113.43 92.06) (end 103.78 92.06) (width 0.27) (layer "F.Cu") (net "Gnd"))
 (segment (start 80.93 128.31) (end 77.21 132.03) (width 0.27) (layer "F.Cu") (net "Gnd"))
 (segment (start 100.82 137.25) (end 100.55 137.25) (width 0.27) (layer "F.Cu") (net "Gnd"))
 (segment (start 100.55 137.25) (end 80.13 137.25) (width 0.27) (layer "F.Cu") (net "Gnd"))
 (segment (start 77.21 135.68) (end 78.72 137.19) (width 0.27) (layer "F.Cu") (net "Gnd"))
 (segment (start 92.69 142.33) (end 82.27 152.75) (width 0.27) (layer "F.Cu") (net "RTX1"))
 (segment (start 73.86 106.64) (end 78.2 102.3) (width 0.27) (layer "F.Cu") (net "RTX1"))
 (segment (start 78.34 152.75) (end 73.86 148.27) (width 0.27) (layer "F.Cu") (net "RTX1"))
 (segment (start 100.55 142.33) (end 92.69 142.33) (width 0.27) (layer "F.Cu") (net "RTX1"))
 (segment (start 82.27 152.75) (end 78.34 152.75) (width 0.27) (layer "F.Cu") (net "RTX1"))
 (segment (start 73.86 148.27) (end 73.86 106.64) (width 0.27) (layer "F.Cu") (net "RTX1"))
 (segment (start 74.77 146.99) (end 74.77 108.27) (width 0.27) (layer "F.Cu") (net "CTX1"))
 (segment (start 100.55 139.79) (end 92.95 139.79) (width 0.27) (layer "F.Cu") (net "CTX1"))
 (segment (start 81.63 151.11) (end 78.89 151.11) (width 0.27) (layer "F.Cu") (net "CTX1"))
 (segment (start 92.95 139.79) (end 81.63 151.11) (width 0.27) (layer "F.Cu") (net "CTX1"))
 (segment (start 78.89 151.11) (end 74.77 146.99) (width 0.27) (layer "F.Cu") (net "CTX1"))
 (segment (start 74.77 108.27) (end 78.2 104.84) (width 0.27) (layer "F.Cu") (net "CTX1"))
 (segment (start 75.83 137.52) (end 75.83 117.37) (width 0.27) (layer "F.Cu") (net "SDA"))
 (segment (start 80.07 141.76) (end 75.83 137.52) (width 0.27) (layer "F.Cu") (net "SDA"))
 (segment (start 75.83 117.37) (end 78.2 115) (width 0.27) (layer "F.Cu") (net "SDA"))
 (segment (start 80.07 142.27) (end 80.07 141.76) (width 0.27) (layer "F.Cu") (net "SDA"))
 (segment (start 80.07 139.73) (end 79.78 139.73) (width 0.27) (layer "F.Cu") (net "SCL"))
 (segment (start 76.44 136.39) (end 76.44 124.38) (width 0.27) (layer "F.Cu") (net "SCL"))
 (segment (start 76.44 124.38) (end 78.2 122.62) (width 0.27) (layer "F.Cu") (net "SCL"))
 (segment (start 79.78 139.73) (end 76.44 136.39) (width 0.27) (layer "F.Cu") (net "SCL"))
 (segment (start 100.55 144.87) (end 125.23 144.87) (width 0.27) (layer "F.Cu") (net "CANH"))
 (segment (start 125.23 144.87) (end 125.28 144.92) (width 0.27) (layer "F.Cu") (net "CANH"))
 (segment (start 100.6 147.46) (end 100.55 147.41) (width 0.27) (layer "F.Cu") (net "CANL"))
 (segment (start 125.28 147.46) (end 100.6 147.46) (width 0.27) (layer "F.Cu") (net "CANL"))
 (segment (start 111.22 127.96) (end 111.22 104.43) (width 0.27) (layer "F.Cu") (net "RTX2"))
 (segment (start 125.55 142.29) (end 111.22 127.96) (width 0.27) (layer "F.Cu") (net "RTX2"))
 (segment (start 111.22 104.43) (end 113.43 102.22) (width 0.27) (layer "F.Cu") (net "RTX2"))
 (segment (start 115.8 107.13) (end 113.43 104.76) (width 0.27) (layer "F.Cu") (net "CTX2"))
 (segment (start 125.55 139.75) (end 115.8 130) (width 0.27) (layer "F.Cu") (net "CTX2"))
 (segment (start 115.8 130) (end 115.8 107.13) (width 0.27) (layer "F.Cu") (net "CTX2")))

